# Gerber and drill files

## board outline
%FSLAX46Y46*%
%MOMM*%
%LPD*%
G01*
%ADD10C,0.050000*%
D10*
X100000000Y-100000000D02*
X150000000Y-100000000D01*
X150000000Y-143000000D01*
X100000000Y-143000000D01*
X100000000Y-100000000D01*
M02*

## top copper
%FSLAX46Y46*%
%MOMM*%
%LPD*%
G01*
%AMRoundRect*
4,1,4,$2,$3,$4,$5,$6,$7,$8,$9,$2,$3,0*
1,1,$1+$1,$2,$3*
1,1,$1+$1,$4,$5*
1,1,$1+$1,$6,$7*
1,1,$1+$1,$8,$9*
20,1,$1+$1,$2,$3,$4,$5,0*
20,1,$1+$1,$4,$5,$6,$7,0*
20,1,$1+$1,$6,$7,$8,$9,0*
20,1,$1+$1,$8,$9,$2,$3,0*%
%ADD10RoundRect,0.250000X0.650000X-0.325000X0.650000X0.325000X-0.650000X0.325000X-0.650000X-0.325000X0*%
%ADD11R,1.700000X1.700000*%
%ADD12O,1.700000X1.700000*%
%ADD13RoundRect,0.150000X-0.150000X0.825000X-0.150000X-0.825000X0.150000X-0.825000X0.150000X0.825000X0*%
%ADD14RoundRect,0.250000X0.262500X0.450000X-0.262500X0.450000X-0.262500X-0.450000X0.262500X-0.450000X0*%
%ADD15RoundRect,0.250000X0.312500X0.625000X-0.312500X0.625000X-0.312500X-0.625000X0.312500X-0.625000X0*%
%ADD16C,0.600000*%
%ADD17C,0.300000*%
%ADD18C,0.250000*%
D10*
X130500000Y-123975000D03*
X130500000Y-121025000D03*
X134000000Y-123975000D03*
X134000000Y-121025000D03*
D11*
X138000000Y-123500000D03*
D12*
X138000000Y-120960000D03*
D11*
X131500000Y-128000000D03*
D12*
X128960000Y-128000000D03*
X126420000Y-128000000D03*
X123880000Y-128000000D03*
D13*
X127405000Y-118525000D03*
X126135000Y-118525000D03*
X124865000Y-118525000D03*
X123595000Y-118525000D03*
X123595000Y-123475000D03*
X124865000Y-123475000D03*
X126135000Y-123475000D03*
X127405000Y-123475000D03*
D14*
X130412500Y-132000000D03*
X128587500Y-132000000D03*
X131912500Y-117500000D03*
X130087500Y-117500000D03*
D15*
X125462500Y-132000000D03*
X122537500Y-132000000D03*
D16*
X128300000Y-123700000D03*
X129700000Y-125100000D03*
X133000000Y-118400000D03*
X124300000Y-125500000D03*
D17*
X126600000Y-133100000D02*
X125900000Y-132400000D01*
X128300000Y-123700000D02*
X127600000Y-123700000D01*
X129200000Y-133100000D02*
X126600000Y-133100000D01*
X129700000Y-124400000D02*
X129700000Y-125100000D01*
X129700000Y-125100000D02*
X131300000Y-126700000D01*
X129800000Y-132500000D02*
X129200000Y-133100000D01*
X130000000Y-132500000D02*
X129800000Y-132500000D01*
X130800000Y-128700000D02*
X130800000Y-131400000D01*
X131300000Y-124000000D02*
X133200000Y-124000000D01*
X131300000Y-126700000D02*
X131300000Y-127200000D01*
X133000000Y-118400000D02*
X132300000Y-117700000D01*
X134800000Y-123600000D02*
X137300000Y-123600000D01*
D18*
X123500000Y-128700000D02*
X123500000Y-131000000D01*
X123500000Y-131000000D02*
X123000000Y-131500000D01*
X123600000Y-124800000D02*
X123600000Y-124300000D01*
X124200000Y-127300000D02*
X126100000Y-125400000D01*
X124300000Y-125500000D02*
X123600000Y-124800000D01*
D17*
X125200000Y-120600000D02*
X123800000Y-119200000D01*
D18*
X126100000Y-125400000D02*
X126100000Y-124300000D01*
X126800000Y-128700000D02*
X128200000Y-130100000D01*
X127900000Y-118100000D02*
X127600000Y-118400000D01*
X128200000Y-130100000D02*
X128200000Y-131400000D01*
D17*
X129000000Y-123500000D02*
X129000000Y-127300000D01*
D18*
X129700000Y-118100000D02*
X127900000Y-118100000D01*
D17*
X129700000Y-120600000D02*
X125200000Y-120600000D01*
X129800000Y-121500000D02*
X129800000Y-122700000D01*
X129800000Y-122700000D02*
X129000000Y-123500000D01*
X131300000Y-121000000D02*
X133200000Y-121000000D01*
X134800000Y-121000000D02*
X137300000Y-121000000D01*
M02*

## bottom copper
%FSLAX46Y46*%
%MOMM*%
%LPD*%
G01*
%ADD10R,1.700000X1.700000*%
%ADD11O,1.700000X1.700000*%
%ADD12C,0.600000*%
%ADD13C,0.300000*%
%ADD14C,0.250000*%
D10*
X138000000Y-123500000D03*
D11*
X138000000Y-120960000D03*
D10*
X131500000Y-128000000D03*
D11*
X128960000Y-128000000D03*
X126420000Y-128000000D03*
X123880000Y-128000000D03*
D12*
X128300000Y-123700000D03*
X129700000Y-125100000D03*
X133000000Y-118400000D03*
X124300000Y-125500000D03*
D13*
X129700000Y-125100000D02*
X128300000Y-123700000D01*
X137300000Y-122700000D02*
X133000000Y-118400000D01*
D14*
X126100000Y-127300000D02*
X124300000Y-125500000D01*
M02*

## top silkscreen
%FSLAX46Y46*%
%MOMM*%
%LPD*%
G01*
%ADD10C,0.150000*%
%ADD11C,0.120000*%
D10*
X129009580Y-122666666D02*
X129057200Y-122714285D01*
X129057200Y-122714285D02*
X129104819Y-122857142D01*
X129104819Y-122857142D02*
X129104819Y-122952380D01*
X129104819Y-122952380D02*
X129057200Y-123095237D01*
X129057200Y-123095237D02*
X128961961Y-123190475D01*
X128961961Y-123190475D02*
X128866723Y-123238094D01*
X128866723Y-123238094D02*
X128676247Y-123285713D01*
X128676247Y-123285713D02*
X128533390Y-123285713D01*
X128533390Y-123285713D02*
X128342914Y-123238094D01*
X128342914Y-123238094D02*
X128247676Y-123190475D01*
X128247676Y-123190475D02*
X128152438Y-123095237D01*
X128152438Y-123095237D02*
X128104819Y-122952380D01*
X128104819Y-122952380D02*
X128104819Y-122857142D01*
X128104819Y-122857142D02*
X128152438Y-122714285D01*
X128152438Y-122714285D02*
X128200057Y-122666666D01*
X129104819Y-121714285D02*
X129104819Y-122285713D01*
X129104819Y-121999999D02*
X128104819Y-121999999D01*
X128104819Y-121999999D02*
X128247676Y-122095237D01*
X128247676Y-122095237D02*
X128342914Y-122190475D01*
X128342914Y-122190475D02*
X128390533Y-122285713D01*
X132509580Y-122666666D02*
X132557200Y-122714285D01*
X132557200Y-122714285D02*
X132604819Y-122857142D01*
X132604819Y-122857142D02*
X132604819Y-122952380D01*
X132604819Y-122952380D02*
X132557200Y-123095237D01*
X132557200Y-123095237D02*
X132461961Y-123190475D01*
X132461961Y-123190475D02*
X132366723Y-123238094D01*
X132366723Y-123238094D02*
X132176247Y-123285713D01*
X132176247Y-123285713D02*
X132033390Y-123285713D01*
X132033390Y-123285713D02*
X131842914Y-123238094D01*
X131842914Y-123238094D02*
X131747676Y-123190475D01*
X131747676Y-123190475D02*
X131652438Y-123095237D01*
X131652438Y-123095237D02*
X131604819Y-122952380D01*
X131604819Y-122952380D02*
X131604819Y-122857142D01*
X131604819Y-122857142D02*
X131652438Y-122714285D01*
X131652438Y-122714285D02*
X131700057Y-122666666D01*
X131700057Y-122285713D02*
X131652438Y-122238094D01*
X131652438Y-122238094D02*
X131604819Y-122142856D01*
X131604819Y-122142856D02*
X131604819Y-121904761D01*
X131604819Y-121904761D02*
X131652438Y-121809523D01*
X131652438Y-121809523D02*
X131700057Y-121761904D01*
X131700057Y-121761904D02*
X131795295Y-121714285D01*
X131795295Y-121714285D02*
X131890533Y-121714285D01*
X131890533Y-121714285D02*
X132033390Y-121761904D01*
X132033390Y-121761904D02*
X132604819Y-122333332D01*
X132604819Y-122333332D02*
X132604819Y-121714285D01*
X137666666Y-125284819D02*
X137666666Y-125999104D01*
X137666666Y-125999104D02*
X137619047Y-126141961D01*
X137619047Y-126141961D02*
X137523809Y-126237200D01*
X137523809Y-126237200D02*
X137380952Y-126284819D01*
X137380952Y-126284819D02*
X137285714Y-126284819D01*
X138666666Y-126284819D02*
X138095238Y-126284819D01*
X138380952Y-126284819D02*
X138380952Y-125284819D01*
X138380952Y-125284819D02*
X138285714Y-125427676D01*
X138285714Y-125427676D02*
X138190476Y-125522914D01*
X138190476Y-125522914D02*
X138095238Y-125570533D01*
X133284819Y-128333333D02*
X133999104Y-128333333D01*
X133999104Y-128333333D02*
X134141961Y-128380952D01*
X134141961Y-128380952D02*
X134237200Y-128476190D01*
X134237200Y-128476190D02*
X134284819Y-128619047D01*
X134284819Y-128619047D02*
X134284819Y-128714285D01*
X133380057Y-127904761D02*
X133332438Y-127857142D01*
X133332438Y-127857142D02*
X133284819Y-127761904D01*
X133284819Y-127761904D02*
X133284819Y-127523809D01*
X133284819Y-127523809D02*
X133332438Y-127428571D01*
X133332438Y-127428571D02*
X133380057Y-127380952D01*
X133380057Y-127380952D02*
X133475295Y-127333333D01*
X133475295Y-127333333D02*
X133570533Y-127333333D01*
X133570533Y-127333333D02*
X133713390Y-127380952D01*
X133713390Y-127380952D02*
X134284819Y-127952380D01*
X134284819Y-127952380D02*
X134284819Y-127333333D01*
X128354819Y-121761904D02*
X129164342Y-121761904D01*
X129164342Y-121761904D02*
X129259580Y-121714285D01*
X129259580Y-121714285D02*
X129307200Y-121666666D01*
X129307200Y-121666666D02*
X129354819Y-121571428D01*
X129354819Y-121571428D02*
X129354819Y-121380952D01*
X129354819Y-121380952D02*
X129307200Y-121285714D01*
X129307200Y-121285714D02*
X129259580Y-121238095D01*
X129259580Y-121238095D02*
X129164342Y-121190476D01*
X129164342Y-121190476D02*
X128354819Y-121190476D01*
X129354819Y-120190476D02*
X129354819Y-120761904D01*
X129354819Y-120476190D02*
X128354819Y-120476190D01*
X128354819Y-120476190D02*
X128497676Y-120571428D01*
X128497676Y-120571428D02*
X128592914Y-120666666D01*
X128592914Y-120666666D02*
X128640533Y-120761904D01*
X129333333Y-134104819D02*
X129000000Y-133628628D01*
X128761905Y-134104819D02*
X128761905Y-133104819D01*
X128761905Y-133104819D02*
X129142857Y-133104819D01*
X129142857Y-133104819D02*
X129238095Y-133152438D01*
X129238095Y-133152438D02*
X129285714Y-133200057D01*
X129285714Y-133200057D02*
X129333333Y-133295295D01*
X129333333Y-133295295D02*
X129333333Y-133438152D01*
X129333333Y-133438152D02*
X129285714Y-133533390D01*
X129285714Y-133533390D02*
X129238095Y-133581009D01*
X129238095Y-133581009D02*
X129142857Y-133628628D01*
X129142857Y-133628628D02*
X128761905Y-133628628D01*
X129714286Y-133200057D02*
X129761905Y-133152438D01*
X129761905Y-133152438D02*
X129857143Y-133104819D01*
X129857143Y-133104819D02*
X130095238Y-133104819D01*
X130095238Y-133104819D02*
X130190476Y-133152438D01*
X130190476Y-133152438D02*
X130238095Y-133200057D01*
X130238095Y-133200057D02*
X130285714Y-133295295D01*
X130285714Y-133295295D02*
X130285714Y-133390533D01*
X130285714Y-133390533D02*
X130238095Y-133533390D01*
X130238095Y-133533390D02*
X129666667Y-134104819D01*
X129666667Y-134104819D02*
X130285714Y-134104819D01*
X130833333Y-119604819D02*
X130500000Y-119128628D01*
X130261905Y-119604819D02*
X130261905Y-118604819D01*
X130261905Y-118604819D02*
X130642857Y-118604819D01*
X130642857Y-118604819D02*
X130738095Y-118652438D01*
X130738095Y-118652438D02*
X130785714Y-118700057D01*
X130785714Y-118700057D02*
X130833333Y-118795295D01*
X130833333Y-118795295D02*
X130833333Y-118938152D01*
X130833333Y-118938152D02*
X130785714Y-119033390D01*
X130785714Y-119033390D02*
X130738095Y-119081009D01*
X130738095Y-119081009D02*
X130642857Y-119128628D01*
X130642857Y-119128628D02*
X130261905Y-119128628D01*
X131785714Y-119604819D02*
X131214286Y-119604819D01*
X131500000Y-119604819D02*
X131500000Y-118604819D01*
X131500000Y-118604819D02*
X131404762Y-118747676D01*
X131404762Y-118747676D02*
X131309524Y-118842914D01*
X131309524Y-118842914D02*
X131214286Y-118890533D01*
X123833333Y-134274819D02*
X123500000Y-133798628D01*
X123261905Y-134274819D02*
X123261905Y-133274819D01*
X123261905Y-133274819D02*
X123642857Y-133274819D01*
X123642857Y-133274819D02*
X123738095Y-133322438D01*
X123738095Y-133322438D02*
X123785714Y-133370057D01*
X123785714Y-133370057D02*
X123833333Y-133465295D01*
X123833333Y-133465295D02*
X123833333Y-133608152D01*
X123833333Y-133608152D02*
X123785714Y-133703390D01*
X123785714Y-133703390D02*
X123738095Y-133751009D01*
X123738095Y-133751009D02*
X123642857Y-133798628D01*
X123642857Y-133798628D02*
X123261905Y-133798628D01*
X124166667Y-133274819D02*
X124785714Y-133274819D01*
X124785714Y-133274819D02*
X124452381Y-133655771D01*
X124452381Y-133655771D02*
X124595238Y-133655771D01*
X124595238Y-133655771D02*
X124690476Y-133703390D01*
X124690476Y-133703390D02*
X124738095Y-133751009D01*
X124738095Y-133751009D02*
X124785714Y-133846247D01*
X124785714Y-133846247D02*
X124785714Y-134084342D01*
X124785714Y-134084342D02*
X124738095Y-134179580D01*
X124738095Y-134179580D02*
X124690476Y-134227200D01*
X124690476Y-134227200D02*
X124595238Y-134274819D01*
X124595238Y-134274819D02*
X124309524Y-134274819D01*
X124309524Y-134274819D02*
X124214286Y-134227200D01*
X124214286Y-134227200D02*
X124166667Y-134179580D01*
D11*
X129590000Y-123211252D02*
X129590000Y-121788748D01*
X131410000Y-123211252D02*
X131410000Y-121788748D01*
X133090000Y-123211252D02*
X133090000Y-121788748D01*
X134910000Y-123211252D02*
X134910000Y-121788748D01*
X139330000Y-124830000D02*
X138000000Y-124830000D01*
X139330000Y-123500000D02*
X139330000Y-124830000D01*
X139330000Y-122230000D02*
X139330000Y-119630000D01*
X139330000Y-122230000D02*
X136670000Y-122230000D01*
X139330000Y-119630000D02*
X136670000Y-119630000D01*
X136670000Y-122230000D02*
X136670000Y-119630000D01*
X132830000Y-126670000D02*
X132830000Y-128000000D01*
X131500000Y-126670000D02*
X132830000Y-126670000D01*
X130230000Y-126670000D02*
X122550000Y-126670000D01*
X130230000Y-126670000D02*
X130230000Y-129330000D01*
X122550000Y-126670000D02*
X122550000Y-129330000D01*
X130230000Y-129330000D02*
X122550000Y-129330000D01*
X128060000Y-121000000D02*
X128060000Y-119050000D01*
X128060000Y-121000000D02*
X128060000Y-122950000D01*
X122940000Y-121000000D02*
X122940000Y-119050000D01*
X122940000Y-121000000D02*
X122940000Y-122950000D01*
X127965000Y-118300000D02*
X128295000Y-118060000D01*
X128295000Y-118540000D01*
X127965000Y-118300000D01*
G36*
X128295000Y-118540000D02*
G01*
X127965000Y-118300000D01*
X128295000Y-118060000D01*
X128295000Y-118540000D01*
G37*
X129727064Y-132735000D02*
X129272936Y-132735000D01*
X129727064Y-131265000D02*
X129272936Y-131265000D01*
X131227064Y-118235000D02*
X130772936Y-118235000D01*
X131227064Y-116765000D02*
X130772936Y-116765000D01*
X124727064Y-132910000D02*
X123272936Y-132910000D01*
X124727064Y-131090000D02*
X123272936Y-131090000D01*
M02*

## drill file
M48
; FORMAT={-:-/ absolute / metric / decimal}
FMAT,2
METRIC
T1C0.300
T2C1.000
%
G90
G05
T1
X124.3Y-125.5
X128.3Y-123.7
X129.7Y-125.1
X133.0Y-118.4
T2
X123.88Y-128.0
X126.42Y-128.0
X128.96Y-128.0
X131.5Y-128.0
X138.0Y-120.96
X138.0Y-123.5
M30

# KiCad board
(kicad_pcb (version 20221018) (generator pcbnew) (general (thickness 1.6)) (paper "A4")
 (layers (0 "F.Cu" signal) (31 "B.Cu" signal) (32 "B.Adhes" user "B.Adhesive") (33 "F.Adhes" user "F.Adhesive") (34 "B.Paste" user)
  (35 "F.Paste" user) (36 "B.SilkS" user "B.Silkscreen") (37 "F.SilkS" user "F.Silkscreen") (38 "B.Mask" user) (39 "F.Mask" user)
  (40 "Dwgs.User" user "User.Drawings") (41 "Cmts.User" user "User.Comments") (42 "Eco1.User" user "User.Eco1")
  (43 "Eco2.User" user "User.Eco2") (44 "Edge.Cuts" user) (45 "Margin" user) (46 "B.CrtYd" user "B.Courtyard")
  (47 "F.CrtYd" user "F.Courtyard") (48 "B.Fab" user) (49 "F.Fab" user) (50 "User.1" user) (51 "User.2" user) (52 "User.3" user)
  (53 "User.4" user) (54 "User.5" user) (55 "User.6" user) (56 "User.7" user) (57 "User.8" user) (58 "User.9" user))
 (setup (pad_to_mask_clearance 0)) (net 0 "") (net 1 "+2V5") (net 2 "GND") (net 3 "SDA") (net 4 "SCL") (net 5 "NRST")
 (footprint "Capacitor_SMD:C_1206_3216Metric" (layer "F.Cu") (at 130.5 122.5 90)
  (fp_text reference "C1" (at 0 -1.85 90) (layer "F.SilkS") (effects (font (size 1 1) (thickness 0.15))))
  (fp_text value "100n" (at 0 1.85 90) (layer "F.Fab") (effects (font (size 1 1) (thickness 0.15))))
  (fp_line (start -0.711252 -0.91) (end 0.711252 -0.91) (stroke (width 0.12) (type solid)) (layer "F.SilkS"))
  (fp_line (start -0.711252 0.91) (end 0.711252 0.91) (stroke (width 0.12) (type solid)) (layer "F.SilkS"))
  (pad "1" smd roundrect (at -1.475 0 90) (size 1.15 1.8) (layers "F.Cu" "F.Paste" "F.Mask") (roundrect_rratio 0.217391) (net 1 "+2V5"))
  (pad "2" smd roundrect (at 1.475 0 90) (size 1.15 1.8) (layers "F.Cu" "F.Paste" "F.Mask") (roundrect_rratio 0.217391) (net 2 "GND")))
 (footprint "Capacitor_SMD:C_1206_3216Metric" (layer "F.Cu") (at 134 122.5 90)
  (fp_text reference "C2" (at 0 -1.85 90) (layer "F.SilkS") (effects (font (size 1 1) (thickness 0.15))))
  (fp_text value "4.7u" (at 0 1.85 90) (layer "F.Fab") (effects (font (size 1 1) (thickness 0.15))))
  (fp_line (start -0.711252 -0.91) (end 0.711252 -0.91) (stroke (width 0.12) (type solid)) (layer "F.SilkS"))
  (fp_line (start -0.711252 0.91) (end 0.711252 0.91) (stroke (width 0.12) (type solid)) (layer "F.SilkS"))
  (pad "1" smd roundrect (at -1.475 0 90) (size 1.15 1.8) (layers "F.Cu" "F.Paste" "F.Mask") (roundrect_rratio 0.217391) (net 1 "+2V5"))
  (pad "2" smd roundrect (at 1.475 0 90) (size 1.15 1.8) (layers "F.Cu" "F.Paste" "F.Mask") (roundrect_rratio 0.217391) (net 2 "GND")))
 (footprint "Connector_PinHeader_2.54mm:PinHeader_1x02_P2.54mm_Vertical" (layer "F.Cu") (at 138 123.5 180)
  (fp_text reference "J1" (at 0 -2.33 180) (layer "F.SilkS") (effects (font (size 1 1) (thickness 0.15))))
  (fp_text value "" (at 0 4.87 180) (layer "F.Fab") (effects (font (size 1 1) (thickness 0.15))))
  (fp_line (start -1.33 -1.33) (end 0 -1.33) (stroke (width 0.12) (type solid)) (layer "F.SilkS"))
  (fp_line (start -1.33 0) (end -1.33 -1.33) (stroke (width 0.12) (type solid)) (layer "F.SilkS"))
  (fp_line (start -1.33 1.27) (end -1.33 3.87) (stroke (width 0.12) (type solid)) (layer "F.SilkS"))
  (fp_line (start -1.33 1.27) (end 1.33 1.27) (stroke (width 0.12) (type solid)) (layer "F.SilkS"))
  (fp_line (start -1.33 3.87) (end 1.33 3.87) (stroke (width 0.12) (type solid)) (layer "F.SilkS"))
  (fp_line (start 1.33 1.27) (end 1.33 3.87) (stroke (width 0.12) (type solid)) (layer "F.SilkS"))
  (pad "1" thru_hole rect (at 0 0 180) (size 1.7 1.7) (drill 1) (layers "*.Cu" "*.Mask") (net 1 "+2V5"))
  (pad "2" thru_hole oval (at 0 2.54 180) (size 1.7 1.7) (drill 1) (layers "*.Cu" "*.Mask") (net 2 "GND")))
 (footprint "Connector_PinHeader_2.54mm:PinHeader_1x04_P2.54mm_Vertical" (layer "F.Cu") (at 131.5 128 -90)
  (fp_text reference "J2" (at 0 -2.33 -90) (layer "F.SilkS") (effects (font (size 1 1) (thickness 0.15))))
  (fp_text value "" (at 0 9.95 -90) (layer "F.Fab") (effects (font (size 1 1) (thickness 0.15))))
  (fp_line (start -1.33 -1.33) (end 0 -1.33) (stroke (width 0.12) (type solid)) (layer "F.SilkS"))
  (fp_line (start -1.33 0) (end -1.33 -1.33) (stroke (width 0.12) (type solid)) (layer "F.SilkS"))
  (fp_line (start -1.33 1.27) (end -1.33 8.95) (stroke (width 0.12) (type solid)) (layer "F.SilkS"))
  (fp_line (start -1.33 1.27) (end 1.33 1.27) (stroke (width 0.12) (type solid)) (layer "F.SilkS"))
  (fp_line (start -1.33 8.95) (end 1.33 8.95) (stroke (width 0.12) (type solid)) (layer "F.SilkS"))
  (fp_line (start 1.33 1.27) (end 1.33 8.95) (stroke (width 0.12) (type solid)) (layer "F.SilkS"))
  (pad "1" thru_hole rect (at 0 0 270) (size 1.7 1.7) (drill 1) (layers "*.Cu" "*.Mask") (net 1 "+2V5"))
  (pad "2" thru_hole oval (at 0 2.54 270) (size 1.7 1.7) (drill 1) (layers "*.Cu" "*.Mask") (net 2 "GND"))
  (pad "3" thru_hole oval (at 0 5.08 270) (size 1.7 1.7) (drill 1) (layers "*.Cu" "*.Mask") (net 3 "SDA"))
  (pad "4" thru_hole oval (at 0 7.62 270) (size 1.7 1.7) (drill 1) (layers "*.Cu" "*.Mask") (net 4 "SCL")))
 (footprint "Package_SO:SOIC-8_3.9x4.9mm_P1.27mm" (layer "F.Cu") (at 125.5 121 -90)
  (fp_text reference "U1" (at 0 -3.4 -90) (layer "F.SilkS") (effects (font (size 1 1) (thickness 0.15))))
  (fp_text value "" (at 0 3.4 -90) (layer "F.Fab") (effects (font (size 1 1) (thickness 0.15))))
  (fp_line (start 0 -2.56) (end -1.95 -2.56) (stroke (width 0.12) (type solid)) (layer "F.SilkS"))
  (fp_line (start 0 -2.56) (end 1.95 -2.56) (stroke (width 0.12) (type solid)) (layer "F.SilkS"))
  (fp_line (start 0 2.56) (end -1.95 2.56) (stroke (width 0.12) (type solid)) (layer "F.SilkS"))
  (fp_line (start 0 2.56) (end 1.95 2.56) (stroke (width 0.12) (type solid)) (layer "F.SilkS"))
  (fp_poly
   (pts (xy -2.7 -2.465) (xy -2.94 -2.795) (xy -2.46 -2.795) (xy -2.7 -2.465)) (stroke (width 0.12) (type solid)) (fill solid)
   (layer "F.SilkS"))
  (pad "1" smd roundrect (at -2.475 -1.905 270) (size 1.95 0.6) (layers "F.Cu" "F.Paste" "F.Mask") (roundrect_rratio 0.25) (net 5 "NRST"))
  (pad "2" smd roundrect (at -2.475 -0.635 270) (size 1.95 0.6) (layers "F.Cu" "F.Paste" "F.Mask") (roundrect_rratio 0.25))
  (pad "3" smd roundrect (at -2.475 0.635 270) (size 1.95 0.6) (layers "F.Cu" "F.Paste" "F.Mask") (roundrect_rratio 0.25))
  (pad "4" smd roundrect (at -2.475 1.905 270) (size 1.95 0.6) (layers "F.Cu" "F.Paste" "F.Mask") (roundrect_rratio 0.25) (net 2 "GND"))
  (pad "5" smd roundrect (at 2.475 1.905 270) (size 1.95 0.6) (layers "F.Cu" "F.Paste" "F.Mask") (roundrect_rratio 0.25) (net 3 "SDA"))
  (pad "6" smd roundrect (at 2.475 0.635 270) (size 1.95 0.6) (layers "F.Cu" "F.Paste" "F.Mask") (roundrect_rratio 0.25))
  (pad "7" smd roundrect (at 2.475 -0.635 270) (size 1.95 0.6) (layers "F.Cu" "F.Paste" "F.Mask") (roundrect_rratio 0.25) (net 4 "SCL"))
  (pad "8" smd roundrect (at 2.475 -1.905 270) (size 1.95 0.6) (layers "F.Cu" "F.Paste" "F.Mask") (roundrect_rratio 0.25) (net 1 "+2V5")))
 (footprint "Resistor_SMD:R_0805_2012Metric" (layer "F.Cu") (at 129.5 132 180)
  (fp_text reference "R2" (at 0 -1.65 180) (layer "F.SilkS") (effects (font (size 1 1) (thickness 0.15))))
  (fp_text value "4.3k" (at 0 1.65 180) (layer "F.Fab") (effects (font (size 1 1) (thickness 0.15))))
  (fp_line (start -0.227064 -0.735) (end 0.227064 -0.735) (stroke (width 0.12) (type solid)) (layer "F.SilkS"))
  (fp_line (start -0.227064 0.735) (end 0.227064 0.735) (stroke (width 0.12) (type solid)) (layer "F.SilkS"))
  (pad "1" smd roundrect (at -0.9125 0 180) (size 1.025 1.4) (layers "F.Cu" "F.Paste" "F.Mask") (roundrect_rratio 0.243902) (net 1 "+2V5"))
  (pad "2" smd roundrect (at 0.9125 0 180) (size 1.025 1.4) (layers "F.Cu" "F.Paste" "F.Mask") (roundrect_rratio 0.243902) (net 3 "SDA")))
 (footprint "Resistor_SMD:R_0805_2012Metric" (layer "F.Cu") (at 131 117.5 180)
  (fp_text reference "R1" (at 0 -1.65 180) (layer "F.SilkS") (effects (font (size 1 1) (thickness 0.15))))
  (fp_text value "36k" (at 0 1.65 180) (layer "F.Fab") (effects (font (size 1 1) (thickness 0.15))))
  (fp_line (start -0.227064 -0.735) (end 0.227064 -0.735) (stroke (width 0.12) (type solid)) (layer "F.SilkS"))
  (fp_line (start -0.227064 0.735) (end 0.227064 0.735) (stroke (width 0.12) (type solid)) (layer "F.SilkS"))
  (pad "1" smd roundrect (at -0.9125 0 180) (size 1.025 1.4) (layers "F.Cu" "F.Paste" "F.Mask") (roundrect_rratio 0.243902) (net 1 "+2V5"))
  (pad "2" smd roundrect (at 0.9125 0 180) (size 1.025 1.4) (layers "F.Cu" "F.Paste" "F.Mask") (roundrect_rratio 0.243902) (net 5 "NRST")))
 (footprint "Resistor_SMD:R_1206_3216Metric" (layer "F.Cu") (at 124 132 180)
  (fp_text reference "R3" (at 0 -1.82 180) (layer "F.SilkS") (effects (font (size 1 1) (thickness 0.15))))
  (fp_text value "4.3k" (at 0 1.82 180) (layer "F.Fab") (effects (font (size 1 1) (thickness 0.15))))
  (fp_line (start -0.727064 -0.91) (end 0.727064 -0.91) (stroke (width 0.12) (type solid)) (layer "F.SilkS"))
  (fp_line (start -0.727064 0.91) (end 0.727064 0.91) (stroke (width 0.12) (type solid)) (layer "F.SilkS"))
  (pad "1" smd roundrect (at -1.4625 0 180) (size 1.125 1.75) (layers "F.Cu" "F.Paste" "F.Mask") (roundrect_rratio 0.222222) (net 1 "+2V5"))
  (pad "2" smd roundrect (at 1.4625 0 180) (size 1.125 1.75) (layers "F.Cu" "F.Paste" "F.Mask") (roundrect_rratio 0.222222) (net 4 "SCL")))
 (gr_rect (start 100 100) (end 150 143) (stroke (width 0.05) (type default)) (fill none) (layer "Edge.Cuts"))
 (segment (start 126.6 133.1) (end 125.9 132.4) (width 0.3) (layer "F.Cu") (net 1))
 (segment (start 128.3 123.7) (end 127.6 123.7) (width 0.3) (layer "F.Cu") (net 1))
 (segment (start 129.2 133.1) (end 126.6 133.1) (width 0.3) (layer "F.Cu") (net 1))
 (segment (start 129.7 124.4) (end 129.7 125.1) (width 0.3) (layer "F.Cu") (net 1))
 (segment (start 129.7 125.1) (end 131.3 126.7) (width 0.3) (layer "F.Cu") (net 1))
 (segment (start 129.8 132.5) (end 129.2 133.1) (width 0.3) (layer "F.Cu") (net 1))
 (segment (start 130 132.5) (end 129.8 132.5) (width 0.3) (layer "F.Cu") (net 1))
 (segment (start 130.8 128.7) (end 130.8 131.4) (width 0.3) (layer "F.Cu") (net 1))
 (segment (start 131.3 124) (end 133.2 124) (width 0.3) (layer "F.Cu") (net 1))
 (segment (start 131.3 126.7) (end 131.3 127.2) (width 0.3) (layer "F.Cu") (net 1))
 (segment (start 133 118.4) (end 132.3 117.7) (width 0.3) (layer "F.Cu") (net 1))
 (segment (start 134.8 123.6) (end 137.3 123.6) (width 0.3) (layer "F.Cu") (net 1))
 (via (at 128.3 123.7) (size 0.6) (drill 0.3) (layers "F.Cu" "B.Cu") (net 1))
 (via (at 129.7 125.1) (size 0.6) (drill 0.3) (layers "F.Cu" "B.Cu") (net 1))
 (via (at 133 118.4) (size 0.6) (drill 0.3) (layers "F.Cu" "B.Cu") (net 1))
 (segment (start 123.5 128.7) (end 123.5 131) (width 0.25) (layer "F.Cu") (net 4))
 (segment (start 123.5 131) (end 123 131.5) (width 0.25) (layer "F.Cu") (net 4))
 (segment (start 123.6 124.8) (end 123.6 124.3) (width 0.25) (layer "F.Cu") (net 3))
 (segment (start 124.2 127.3) (end 126.1 125.4) (width 0.25) (layer "F.Cu") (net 4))
 (segment (start 124.3 125.5) (end 123.6 124.8) (width 0.25) (layer "F.Cu") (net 3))
 (segment (start 125.2 120.6) (end 123.8 119.2) (width 0.3) (layer "F.Cu") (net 2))
 (segment (start 126.1 125.4) (end 126.1 124.3) (width 0.25) (layer "F.Cu") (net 4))
 (segment (start 126.8 128.7) (end 128.2 130.1) (width 0.25) (layer "F.Cu") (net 3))
 (segment (start 127.9 118.1) (end 127.6 118.4) (width 0.25) (layer "F.Cu") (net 5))
 (segment (start 128.2 130.1) (end 128.2 131.4) (width 0.25) (layer "F.Cu") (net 3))
 (segment (start 129 123.5) (end 129 127.3) (width 0.3) (layer "F.Cu") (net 2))
 (segment (start 129.7 118.1) (end 127.9 118.1) (width 0.25) (layer "F.Cu") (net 5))
 (segment (start 129.7 120.6) (end 125.2 120.6) (width 0.3) (layer "F.Cu") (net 2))
 (segment (start 129.7 125.1) (end 128.3 123.7) (width 0.3) (layer "B.Cu") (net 1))
 (segment (start 129.8 121.5) (end 129.8 122.7) (width 0.3) (layer "F.Cu") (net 2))
 (segment (start 129.8 122.7) (end 129 123.5) (width 0.3) (layer "F.Cu") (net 2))
 (segment (start 131.3 121) (end 133.2 121) (width 0.3) (layer "F.Cu") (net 2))
 (segment (start 134.8 121) (end 137.3 121) (width 0.3) (layer "F.Cu") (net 2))
 (segment (start 137.3 122.7) (end 133 118.4) (width 0.3) (layer "B.Cu") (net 1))
 (via (at 124.3 125.5) (size 0.6) (drill 0.3) (layers "F.Cu" "B.Cu") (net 3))
 (segment (start 126.1 127.3) (end 124.3 125.5) (width 0.25) (layer "B.Cu") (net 3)))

